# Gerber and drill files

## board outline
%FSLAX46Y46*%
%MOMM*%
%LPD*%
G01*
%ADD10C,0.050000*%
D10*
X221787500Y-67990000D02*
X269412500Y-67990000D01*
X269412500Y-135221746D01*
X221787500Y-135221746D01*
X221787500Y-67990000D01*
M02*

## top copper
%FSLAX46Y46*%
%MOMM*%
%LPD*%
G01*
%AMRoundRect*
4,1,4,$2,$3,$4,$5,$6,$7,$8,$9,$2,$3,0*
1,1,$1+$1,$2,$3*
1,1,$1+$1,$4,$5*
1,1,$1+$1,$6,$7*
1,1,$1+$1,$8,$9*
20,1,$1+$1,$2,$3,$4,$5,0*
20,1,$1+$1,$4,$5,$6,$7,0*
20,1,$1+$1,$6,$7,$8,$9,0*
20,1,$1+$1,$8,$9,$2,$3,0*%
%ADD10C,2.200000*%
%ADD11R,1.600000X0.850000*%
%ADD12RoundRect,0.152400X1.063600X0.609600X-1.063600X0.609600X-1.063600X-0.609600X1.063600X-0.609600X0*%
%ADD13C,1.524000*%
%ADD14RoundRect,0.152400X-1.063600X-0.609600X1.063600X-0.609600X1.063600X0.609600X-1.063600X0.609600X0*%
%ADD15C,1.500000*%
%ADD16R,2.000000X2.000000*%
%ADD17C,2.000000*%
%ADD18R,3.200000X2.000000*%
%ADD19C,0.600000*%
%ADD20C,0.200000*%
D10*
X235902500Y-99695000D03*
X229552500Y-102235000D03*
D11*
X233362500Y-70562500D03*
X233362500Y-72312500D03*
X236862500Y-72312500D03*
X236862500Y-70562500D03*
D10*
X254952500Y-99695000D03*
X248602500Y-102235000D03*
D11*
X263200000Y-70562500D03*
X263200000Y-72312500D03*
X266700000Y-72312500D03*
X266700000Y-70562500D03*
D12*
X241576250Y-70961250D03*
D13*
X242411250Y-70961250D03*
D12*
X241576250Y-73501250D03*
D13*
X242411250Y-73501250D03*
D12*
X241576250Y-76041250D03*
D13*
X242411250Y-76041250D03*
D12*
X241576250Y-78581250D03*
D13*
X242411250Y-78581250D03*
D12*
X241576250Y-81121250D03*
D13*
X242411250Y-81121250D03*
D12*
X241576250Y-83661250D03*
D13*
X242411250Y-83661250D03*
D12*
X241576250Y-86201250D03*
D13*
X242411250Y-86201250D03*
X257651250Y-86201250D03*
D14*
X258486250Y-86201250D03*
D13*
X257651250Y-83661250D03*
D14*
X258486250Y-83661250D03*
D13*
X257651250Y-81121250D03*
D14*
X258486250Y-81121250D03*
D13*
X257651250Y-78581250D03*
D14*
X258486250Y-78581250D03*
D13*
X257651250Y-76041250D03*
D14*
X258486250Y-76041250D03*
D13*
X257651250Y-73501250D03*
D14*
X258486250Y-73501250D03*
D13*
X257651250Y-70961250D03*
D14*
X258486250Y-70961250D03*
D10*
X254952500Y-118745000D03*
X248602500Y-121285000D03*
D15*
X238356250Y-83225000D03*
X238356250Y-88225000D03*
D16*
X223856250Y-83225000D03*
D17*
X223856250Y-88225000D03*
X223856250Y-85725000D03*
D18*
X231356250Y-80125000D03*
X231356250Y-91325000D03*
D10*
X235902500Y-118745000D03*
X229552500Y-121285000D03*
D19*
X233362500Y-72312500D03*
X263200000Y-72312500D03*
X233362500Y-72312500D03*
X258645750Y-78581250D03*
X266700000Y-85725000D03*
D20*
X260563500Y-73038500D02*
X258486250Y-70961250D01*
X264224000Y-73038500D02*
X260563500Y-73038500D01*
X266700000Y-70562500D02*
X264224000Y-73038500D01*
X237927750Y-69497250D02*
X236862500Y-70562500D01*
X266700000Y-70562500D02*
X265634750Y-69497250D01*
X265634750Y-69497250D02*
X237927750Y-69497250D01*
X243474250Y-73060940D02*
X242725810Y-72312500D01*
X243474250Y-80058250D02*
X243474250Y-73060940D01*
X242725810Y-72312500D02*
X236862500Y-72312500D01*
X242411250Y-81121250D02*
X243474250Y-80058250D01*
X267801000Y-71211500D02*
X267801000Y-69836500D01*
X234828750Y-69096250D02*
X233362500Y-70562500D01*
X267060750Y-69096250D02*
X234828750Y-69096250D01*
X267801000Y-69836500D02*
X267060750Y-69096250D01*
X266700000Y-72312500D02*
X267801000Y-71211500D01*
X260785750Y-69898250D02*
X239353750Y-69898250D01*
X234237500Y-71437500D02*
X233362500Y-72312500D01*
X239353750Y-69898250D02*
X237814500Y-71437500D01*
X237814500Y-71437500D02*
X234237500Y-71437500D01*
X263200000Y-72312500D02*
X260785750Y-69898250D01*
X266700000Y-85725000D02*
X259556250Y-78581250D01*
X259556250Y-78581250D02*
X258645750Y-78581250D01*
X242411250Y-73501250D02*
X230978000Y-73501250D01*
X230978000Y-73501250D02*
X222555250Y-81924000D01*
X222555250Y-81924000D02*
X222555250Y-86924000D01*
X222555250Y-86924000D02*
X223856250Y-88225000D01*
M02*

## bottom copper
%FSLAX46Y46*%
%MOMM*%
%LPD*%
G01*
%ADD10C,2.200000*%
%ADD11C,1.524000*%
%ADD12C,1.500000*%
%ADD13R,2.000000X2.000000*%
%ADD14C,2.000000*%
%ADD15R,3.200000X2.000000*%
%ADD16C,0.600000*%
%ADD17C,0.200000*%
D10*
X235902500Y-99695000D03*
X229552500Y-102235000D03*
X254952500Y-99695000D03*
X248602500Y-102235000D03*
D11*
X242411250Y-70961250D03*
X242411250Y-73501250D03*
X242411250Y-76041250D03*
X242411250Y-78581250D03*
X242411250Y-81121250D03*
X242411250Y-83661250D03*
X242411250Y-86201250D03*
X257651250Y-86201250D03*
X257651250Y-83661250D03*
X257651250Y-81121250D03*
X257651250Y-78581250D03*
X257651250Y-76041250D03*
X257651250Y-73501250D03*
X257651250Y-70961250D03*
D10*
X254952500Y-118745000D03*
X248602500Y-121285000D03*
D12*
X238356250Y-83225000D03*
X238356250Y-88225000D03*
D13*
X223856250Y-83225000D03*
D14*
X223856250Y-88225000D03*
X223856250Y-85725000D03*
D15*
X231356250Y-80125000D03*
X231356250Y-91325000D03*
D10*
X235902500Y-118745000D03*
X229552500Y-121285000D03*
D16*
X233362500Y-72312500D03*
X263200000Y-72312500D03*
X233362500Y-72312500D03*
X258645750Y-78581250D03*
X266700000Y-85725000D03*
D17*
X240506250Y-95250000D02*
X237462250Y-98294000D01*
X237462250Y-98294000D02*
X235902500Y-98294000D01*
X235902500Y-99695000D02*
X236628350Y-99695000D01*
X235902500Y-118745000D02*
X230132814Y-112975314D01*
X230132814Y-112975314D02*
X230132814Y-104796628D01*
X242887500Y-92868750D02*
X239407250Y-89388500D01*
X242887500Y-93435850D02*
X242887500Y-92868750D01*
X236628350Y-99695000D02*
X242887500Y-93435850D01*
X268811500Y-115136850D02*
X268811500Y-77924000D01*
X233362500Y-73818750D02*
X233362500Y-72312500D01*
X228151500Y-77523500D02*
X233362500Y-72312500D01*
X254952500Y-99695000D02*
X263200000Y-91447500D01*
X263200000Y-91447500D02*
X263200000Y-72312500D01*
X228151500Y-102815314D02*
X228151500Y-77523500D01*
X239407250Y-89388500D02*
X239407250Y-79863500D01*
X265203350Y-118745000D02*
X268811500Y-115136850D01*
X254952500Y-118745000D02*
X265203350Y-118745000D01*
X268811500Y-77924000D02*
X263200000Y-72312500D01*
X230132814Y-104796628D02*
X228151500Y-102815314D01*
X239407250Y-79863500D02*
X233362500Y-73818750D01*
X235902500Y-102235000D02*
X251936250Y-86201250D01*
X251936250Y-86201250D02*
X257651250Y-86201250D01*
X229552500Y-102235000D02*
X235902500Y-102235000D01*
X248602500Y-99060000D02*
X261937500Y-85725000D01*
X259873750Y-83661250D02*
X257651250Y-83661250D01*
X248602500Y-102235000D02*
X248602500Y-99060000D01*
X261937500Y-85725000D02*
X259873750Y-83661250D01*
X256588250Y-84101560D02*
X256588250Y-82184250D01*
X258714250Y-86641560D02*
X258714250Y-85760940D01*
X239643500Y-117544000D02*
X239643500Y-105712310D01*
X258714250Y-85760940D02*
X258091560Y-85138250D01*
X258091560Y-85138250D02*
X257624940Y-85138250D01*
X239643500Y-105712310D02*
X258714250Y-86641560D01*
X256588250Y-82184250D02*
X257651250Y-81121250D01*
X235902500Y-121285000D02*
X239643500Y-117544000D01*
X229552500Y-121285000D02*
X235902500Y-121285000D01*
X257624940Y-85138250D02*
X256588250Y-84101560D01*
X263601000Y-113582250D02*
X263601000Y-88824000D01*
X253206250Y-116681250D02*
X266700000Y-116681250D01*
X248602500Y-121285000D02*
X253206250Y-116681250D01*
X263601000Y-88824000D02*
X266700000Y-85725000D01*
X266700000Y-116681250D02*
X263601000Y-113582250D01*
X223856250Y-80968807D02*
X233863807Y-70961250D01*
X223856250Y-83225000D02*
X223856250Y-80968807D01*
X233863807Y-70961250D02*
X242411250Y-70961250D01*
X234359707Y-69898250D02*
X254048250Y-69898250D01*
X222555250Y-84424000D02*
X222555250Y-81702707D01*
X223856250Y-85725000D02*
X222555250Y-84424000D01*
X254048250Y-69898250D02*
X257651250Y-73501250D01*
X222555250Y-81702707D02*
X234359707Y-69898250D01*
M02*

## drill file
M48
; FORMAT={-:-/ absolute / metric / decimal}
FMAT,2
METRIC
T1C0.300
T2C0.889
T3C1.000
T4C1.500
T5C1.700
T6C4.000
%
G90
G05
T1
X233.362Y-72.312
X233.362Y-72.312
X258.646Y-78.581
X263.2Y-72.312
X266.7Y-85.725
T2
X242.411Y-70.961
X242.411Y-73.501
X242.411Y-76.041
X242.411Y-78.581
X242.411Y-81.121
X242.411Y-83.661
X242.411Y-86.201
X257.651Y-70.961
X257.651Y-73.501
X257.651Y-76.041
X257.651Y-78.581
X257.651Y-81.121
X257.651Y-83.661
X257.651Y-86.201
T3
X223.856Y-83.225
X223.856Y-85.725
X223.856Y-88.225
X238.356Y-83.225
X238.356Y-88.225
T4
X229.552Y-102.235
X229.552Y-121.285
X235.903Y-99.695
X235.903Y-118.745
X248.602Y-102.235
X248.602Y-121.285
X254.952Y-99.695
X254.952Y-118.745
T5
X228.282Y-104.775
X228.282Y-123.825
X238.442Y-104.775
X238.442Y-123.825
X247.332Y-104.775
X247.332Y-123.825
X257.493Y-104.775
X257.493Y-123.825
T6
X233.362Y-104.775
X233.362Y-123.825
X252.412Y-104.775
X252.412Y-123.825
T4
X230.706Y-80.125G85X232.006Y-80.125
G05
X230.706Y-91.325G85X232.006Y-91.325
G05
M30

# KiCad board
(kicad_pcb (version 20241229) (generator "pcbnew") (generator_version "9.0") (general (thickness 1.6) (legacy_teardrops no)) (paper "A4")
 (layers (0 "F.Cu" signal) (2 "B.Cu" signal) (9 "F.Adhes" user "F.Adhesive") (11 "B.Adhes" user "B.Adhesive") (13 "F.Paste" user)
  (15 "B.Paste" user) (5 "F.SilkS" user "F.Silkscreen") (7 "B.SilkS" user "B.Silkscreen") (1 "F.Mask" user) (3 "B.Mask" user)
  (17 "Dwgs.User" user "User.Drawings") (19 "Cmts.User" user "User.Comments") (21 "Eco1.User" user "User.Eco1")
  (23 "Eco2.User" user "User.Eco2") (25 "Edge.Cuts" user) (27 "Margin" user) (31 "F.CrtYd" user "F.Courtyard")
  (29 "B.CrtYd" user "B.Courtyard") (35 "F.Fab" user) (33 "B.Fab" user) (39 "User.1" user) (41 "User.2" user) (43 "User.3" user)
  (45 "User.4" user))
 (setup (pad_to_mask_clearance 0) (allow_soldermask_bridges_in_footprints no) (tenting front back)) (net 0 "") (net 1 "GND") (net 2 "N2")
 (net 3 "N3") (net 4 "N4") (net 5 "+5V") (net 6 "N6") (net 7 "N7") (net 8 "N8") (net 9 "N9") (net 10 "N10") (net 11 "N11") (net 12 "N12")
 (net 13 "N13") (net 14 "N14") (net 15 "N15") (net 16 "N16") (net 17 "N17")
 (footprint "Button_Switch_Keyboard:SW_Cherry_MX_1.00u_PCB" (layer "F.Cu") (at 235.9025 99.695)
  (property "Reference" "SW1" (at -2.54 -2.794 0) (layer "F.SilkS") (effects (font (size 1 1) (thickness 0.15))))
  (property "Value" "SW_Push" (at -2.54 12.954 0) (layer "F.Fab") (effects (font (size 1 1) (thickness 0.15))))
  (pad "" np_thru_hole circle (at -7.62 5.08) (size 1.7 1.7) (drill 1.7) (layers "*.Cu" "*.Mask"))
  (pad "" np_thru_hole circle (at -2.54 5.08) (size 4 4) (drill 4) (layers "*.Cu" "*.Mask"))
  (pad "" np_thru_hole circle (at 2.54 5.08) (size 1.7 1.7) (drill 1.7) (layers "*.Cu" "*.Mask"))
  (pad "1" thru_hole circle (at 0 0) (size 2.2 2.2) (drill 1.5) (layers "*.Cu" "*.Mask") (remove_unused_layers no) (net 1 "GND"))
  (pad "2" thru_hole circle (at -6.35 2.54) (size 2.2 2.2) (drill 1.5) (layers "*.Cu" "*.Mask") (remove_unused_layers no) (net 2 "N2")))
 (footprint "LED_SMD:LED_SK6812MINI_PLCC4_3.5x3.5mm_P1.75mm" (layer "F.Cu") (at 235.1125 71.4375)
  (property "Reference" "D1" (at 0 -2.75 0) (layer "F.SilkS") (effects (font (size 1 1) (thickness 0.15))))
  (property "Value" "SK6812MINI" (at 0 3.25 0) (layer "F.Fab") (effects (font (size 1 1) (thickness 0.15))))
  (pad "1" smd rect (at -1.75 -0.875) (size 1.6 0.85) (layers "F.Cu" "F.Mask" "F.Paste") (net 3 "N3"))
  (pad "2" smd rect (at -1.75 0.875) (size 1.6 0.85) (layers "F.Cu" "F.Mask" "F.Paste") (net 1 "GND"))
  (pad "3" smd rect (at 1.75 0.875) (size 1.6 0.85) (layers "F.Cu" "F.Mask" "F.Paste") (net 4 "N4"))
  (pad "4" smd rect (at 1.75 -0.875) (size 1.6 0.85) (layers "F.Cu" "F.Mask" "F.Paste") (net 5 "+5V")))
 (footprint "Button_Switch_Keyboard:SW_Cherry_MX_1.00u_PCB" (layer "F.Cu") (at 254.9525 99.695)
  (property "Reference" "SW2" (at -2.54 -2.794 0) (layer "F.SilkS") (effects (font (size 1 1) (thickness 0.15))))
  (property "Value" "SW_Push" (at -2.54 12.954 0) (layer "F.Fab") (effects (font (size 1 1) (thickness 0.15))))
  (pad "" np_thru_hole circle (at -7.62 5.08) (size 1.7 1.7) (drill 1.7) (layers "*.Cu" "*.Mask"))
  (pad "" np_thru_hole circle (at -2.54 5.08) (size 4 4) (drill 4) (layers "*.Cu" "*.Mask"))
  (pad "" np_thru_hole circle (at 2.54 5.08) (size 1.7 1.7) (drill 1.7) (layers "*.Cu" "*.Mask"))
  (pad "1" thru_hole circle (at 0 0) (size 2.2 2.2) (drill 1.5) (layers "*.Cu" "*.Mask") (remove_unused_layers no) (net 1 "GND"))
  (pad "2" thru_hole circle (at -6.35 2.54) (size 2.2 2.2) (drill 1.5) (layers "*.Cu" "*.Mask") (remove_unused_layers no) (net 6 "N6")))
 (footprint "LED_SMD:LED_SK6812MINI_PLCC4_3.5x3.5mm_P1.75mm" (layer "F.Cu") (at 264.95 71.4375)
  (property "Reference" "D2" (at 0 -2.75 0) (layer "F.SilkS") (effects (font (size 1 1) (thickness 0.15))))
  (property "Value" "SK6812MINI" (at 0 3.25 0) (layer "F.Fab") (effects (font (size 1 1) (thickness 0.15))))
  (pad "1" smd rect (at -1.75 -0.875) (size 1.6 0.85) (layers "F.Cu" "F.Mask" "F.Paste") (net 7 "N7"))
  (pad "2" smd rect (at -1.75 0.875) (size 1.6 0.85) (layers "F.Cu" "F.Mask" "F.Paste") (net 1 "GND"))
  (pad "3" smd rect (at 1.75 0.875) (size 1.6 0.85) (layers "F.Cu" "F.Mask" "F.Paste") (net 3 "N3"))
  (pad "4" smd rect (at 1.75 -0.875) (size 1.6 0.85) (layers "F.Cu" "F.Mask" "F.Paste") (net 5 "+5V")))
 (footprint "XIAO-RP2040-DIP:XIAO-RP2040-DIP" (layer "F.Cu") (at 250.03125 78.58125)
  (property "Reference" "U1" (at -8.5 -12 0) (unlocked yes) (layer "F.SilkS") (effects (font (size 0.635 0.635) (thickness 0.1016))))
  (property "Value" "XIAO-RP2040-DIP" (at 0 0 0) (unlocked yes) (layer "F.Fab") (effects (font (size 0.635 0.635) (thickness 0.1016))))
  (pad "1" smd roundrect (at -8.455 -7.62 180) (size 2.432 1.524) (layers "F.Cu" "F.Mask") (roundrect_rratio 0.1) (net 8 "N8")
   (thermal_bridge_angle 45))
  (pad "1" thru_hole circle (at -7.62 -7.62 180) (size 1.524 1.524) (drill 0.889) (layers "*.Cu" "*.Mask") (remove_unused_layers no)
   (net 8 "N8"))
  (pad "2" smd roundrect (at -8.455 -5.08 180) (size 2.432 1.524) (layers "F.Cu" "F.Mask") (roundrect_rratio 0.1) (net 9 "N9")
   (thermal_bridge_angle 45))
  (pad "2" thru_hole circle (at -7.62 -5.08 180) (size 1.524 1.524) (drill 0.889) (layers "*.Cu" "*.Mask") (remove_unused_layers no)
   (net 9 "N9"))
  (pad "3" smd roundrect (at -8.455 -2.54 180) (size 2.432 1.524) (layers "F.Cu" "F.Mask") (roundrect_rratio 0.1) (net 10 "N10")
   (thermal_bridge_angle 45))
  (pad "3" thru_hole circle (at -7.62 -2.54 180) (size 1.524 1.524) (drill 0.889) (layers "*.Cu" "*.Mask") (remove_unused_layers no)
   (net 10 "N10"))
  (pad "4" smd roundrect (at -8.455 0 180) (size 2.432 1.524) (layers "F.Cu" "F.Mask") (roundrect_rratio 0.1) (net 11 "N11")
   (thermal_bridge_angle 45))
  (pad "4" thru_hole circle (at -7.62 0 180) (size 1.524 1.524) (drill 0.889) (layers "*.Cu" "*.Mask") (remove_unused_layers no)
   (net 11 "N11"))
  (pad "5" smd roundrect (at -8.455 2.54 180) (size 2.432 1.524) (layers "F.Cu" "F.Mask") (roundrect_rratio 0.1) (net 4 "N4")
   (thermal_bridge_angle 45))
  (pad "5" thru_hole circle (at -7.62 2.54 180) (size 1.524 1.524) (drill 0.889) (layers "*.Cu" "*.Mask") (remove_unused_layers no)
   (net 4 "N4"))
  (pad "6" smd roundrect (at -8.455 5.08 180) (size 2.432 1.524) (layers "F.Cu" "F.Mask") (roundrect_rratio 0.1) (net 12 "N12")
   (thermal_bridge_angle 45))
  (pad "6" thru_hole circle (at -7.62 5.08 180) (size 1.524 1.524) (drill 0.889) (layers "*.Cu" "*.Mask") (remove_unused_layers no)
   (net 12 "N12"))
  (pad "7" smd roundrect (at -8.455 7.62 180) (size 2.432 1.524) (layers "F.Cu" "F.Mask") (roundrect_rratio 0.1) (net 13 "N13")
   (thermal_bridge_angle 45))
  (pad "7" thru_hole circle (at -7.62 7.62 180) (size 1.524 1.524) (drill 0.889) (layers "*.Cu" "*.Mask") (remove_unused_layers no)
   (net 13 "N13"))
  (pad "8" thru_hole circle (at 7.62 7.62) (size 1.524 1.524) (drill 0.889) (layers "*.Cu" "*.Mask") (remove_unused_layers no) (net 2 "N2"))
  (pad "8" smd roundrect (at 8.455 7.62) (size 2.432 1.524) (layers "F.Cu" "F.Mask") (roundrect_rratio 0.1) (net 2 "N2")
   (thermal_bridge_angle 45))
  (pad "9" thru_hole circle (at 7.62 5.08) (size 1.524 1.524) (drill 0.889) (layers "*.Cu" "*.Mask") (remove_unused_layers no) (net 6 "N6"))
  (pad "9" smd roundrect (at 8.455 5.08) (size 2.432 1.524) (layers "F.Cu" "F.Mask") (roundrect_rratio 0.1) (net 6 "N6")
   (thermal_bridge_angle 45))
  (pad "10" thru_hole circle (at 7.62 2.54) (size 1.524 1.524) (drill 0.889) (layers "*.Cu" "*.Mask") (remove_unused_layers no)
   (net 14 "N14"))
  (pad "10" smd roundrect (at 8.455 2.54) (size 2.432 1.524) (layers "F.Cu" "F.Mask") (roundrect_rratio 0.1) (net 14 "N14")
   (thermal_bridge_angle 45))
  (pad "11" thru_hole circle (at 7.62 0) (size 1.524 1.524) (drill 0.889) (layers "*.Cu" "*.Mask") (remove_unused_layers no) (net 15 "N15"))
  (pad "11" smd roundrect (at 8.455 0) (size 2.432 1.524) (layers "F.Cu" "F.Mask") (roundrect_rratio 0.1) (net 15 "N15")
   (thermal_bridge_angle 45))
  (pad "12" thru_hole circle (at 7.62 -2.54) (size 1.524 1.524) (drill 0.889) (layers "*.Cu" "*.Mask") (remove_unused_layers no)
   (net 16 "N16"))
  (pad "12" smd roundrect (at 8.455 -2.54) (size 2.432 1.524) (layers "F.Cu" "F.Mask") (roundrect_rratio 0.1) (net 16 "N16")
   (thermal_bridge_angle 45))
  (pad "13" thru_hole circle (at 7.62 -5.08) (size 1.524 1.524) (drill 0.889) (layers "*.Cu" "*.Mask") (remove_unused_layers no)
   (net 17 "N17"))
  (pad "13" smd roundrect (at 8.455 -5.08) (size 2.432 1.524) (layers "F.Cu" "F.Mask") (roundrect_rratio 0.1) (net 17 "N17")
   (thermal_bridge_angle 45))
  (pad "14" thru_hole circle (at 7.62 -7.62) (size 1.524 1.524) (drill 0.889) (layers "*.Cu" "*.Mask") (remove_unused_layers no)
   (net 5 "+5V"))
  (pad "14" smd roundrect (at 8.455 -7.62) (size 2.432 1.524) (layers "F.Cu" "F.Mask") (roundrect_rratio 0.1) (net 5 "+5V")
   (thermal_bridge_angle 45)))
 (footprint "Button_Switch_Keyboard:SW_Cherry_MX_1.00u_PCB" (layer "F.Cu") (at 254.9525 118.745)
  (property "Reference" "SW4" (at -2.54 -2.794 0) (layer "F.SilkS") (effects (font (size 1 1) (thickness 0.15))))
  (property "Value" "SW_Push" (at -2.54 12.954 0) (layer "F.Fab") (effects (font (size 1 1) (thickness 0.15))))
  (pad "" np_thru_hole circle (at -7.62 5.08) (size 1.7 1.7) (drill 1.7) (layers "*.Cu" "*.Mask"))
  (pad "" np_thru_hole circle (at -2.54 5.08) (size 4 4) (drill 4) (layers "*.Cu" "*.Mask"))
  (pad "" np_thru_hole circle (at 2.54 5.08) (size 1.7 1.7) (drill 1.7) (layers "*.Cu" "*.Mask"))
  (pad "1" thru_hole circle (at 0 0) (size 2.2 2.2) (drill 1.5) (layers "*.Cu" "*.Mask") (remove_unused_layers no) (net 1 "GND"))
  (pad "2" thru_hole circle (at -6.35 2.54) (size 2.2 2.2) (drill 1.5) (layers "*.Cu" "*.Mask") (remove_unused_layers no) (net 15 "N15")))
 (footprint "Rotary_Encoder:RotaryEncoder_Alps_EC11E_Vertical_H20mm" (layer "F.Cu") (at 223.85625 83.225)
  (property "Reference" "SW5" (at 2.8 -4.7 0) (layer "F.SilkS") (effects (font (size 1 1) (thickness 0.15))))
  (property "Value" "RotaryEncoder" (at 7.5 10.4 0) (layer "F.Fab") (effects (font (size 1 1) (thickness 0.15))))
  (pad "" thru_hole circle (at 14.5 0) (size 1.5 1.5) (drill 1) (layers "*.Cu" "*.Mask") (remove_unused_layers no))
  (pad "" thru_hole circle (at 14.5 5) (size 1.5 1.5) (drill 1) (layers "*.Cu" "*.Mask") (remove_unused_layers no))
  (pad "A" thru_hole rect (at 0 0) (size 2 2) (drill 1) (layers "*.Cu" "*.Mask") (remove_unused_layers no) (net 8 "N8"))
  (pad "B" thru_hole circle (at 0 5) (size 2 2) (drill 1) (layers "*.Cu" "*.Mask") (remove_unused_layers no) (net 9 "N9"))
  (pad "C" thru_hole circle (at 0 2.5) (size 2 2) (drill 1) (layers "*.Cu" "*.Mask") (remove_unused_layers no) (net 17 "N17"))
  (pad "MP" thru_hole rect (at 7.5 -3.1) (size 3.2 2) (drill oval 2.8 1.5) (layers "*.Cu" "*.Mask") (remove_unused_layers no))
  (pad "MP" thru_hole rect (at 7.5 8.1) (size 3.2 2) (drill oval 2.8 1.5) (layers "*.Cu" "*.Mask") (remove_unused_layers no)))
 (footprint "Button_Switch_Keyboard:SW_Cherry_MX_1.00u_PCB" (layer "F.Cu") (at 235.9025 118.745)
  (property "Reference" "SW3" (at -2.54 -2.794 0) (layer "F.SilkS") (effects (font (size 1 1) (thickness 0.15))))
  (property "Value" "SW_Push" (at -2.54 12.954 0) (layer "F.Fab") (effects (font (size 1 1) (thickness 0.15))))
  (pad "" np_thru_hole circle (at -7.62 5.08) (size 1.7 1.7) (drill 1.7) (layers "*.Cu" "*.Mask"))
  (pad "" np_thru_hole circle (at -2.54 5.08) (size 4 4) (drill 4) (layers "*.Cu" "*.Mask"))
  (pad "" np_thru_hole circle (at 2.54 5.08) (size 1.7 1.7) (drill 1.7) (layers "*.Cu" "*.Mask"))
  (pad "1" thru_hole circle (at 0 0) (size 2.2 2.2) (drill 1.5) (layers "*.Cu" "*.Mask") (remove_unused_layers no) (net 1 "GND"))
  (pad "2" thru_hole circle (at -6.35 2.54) (size 2.2 2.2) (drill 1.5) (layers "*.Cu" "*.Mask") (remove_unused_layers no) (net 14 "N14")))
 (gr_rect (start 221.7875 67.99) (end 269.4125 135.221746) (stroke (width 0.05) (type default)) (fill no) (layer "Edge.Cuts"))
 (segment (start 240.50625 95.25) (end 237.46225 98.294) (width 0.2) (layer "B.Cu") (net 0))
 (segment (start 237.46225 98.294) (end 235.9025 98.294) (width 0.2) (layer "B.Cu") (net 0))
 (segment (start 260.5635 73.0385) (end 258.48625 70.96125) (width 0.2) (layer "F.Cu") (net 5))
 (segment (start 264.224 73.0385) (end 260.5635 73.0385) (width 0.2) (layer "F.Cu") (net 5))
 (segment (start 266.7 70.5625) (end 264.224 73.0385) (width 0.2) (layer "F.Cu") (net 5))
 (segment (start 237.92775 69.49725) (end 236.8625 70.5625) (width 0.2) (layer "F.Cu") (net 5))
 (segment (start 266.7 70.5625) (end 265.63475 69.49725) (width 0.2) (layer "F.Cu") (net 5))
 (segment (start 265.63475 69.49725) (end 237.92775 69.49725) (width 0.2) (layer "F.Cu") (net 5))
 (segment (start 243.47425 73.06094) (end 242.72581 72.3125) (width 0.2) (layer "F.Cu") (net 4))
 (segment (start 243.47425 80.05825) (end 243.47425 73.06094) (width 0.2) (layer "F.Cu") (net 4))
 (segment (start 242.72581 72.3125) (end 236.8625 72.3125) (width 0.2) (layer "F.Cu") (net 4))
 (segment (start 242.41125 81.12125) (end 243.47425 80.05825) (width 0.2) (layer "F.Cu") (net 4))
 (segment (start 267.801 71.2115) (end 267.801 69.8365) (width 0.2) (layer "F.Cu") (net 3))
 (segment (start 234.82875 69.09625) (end 233.3625 70.5625) (width 0.2) (layer "F.Cu") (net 3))
 (segment (start 267.06075 69.09625) (end 234.82875 69.09625) (width 0.2) (layer "F.Cu") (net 3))
 (segment (start 267.801 69.8365) (end 267.06075 69.09625) (width 0.2) (layer "F.Cu") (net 3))
 (segment (start 266.7 72.3125) (end 267.801 71.2115) (width 0.2) (layer "F.Cu") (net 3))
 (segment (start 260.78575 69.89825) (end 239.35375 69.89825) (width 0.2) (layer "F.Cu") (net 1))
 (segment (start 234.2375 71.4375) (end 233.3625 72.3125) (width 0.2) (layer "F.Cu") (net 1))
 (segment (start 239.35375 69.89825) (end 237.8145 71.4375) (width 0.2) (layer "F.Cu") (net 1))
 (segment (start 237.8145 71.4375) (end 234.2375 71.4375) (width 0.2) (layer "F.Cu") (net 1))
 (segment (start 263.2 72.3125) (end 260.78575 69.89825) (width 0.2) (layer "F.Cu") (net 1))
 (via (at 233.3625 72.3125) (size 0.6) (drill 0.3) (layers "F.Cu" "B.Cu") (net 1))
 (via (at 263.2 72.3125) (size 0.6) (drill 0.3) (layers "F.Cu" "B.Cu") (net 1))
 (via (at 233.3625 72.3125) (size 0.6) (drill 0.3) (layers "F.Cu" "B.Cu") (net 1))
 (segment (start 235.9025 99.695) (end 236.62835 99.695) (width 0.2) (layer "B.Cu") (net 1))
 (segment (start 235.9025 118.745) (end 230.132814 112.975314) (width 0.2) (layer "B.Cu") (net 1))
 (segment (start 230.132814 112.975314) (end 230.132814 104.796628) (width 0.2) (layer "B.Cu") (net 1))
 (segment (start 242.8875 92.86875) (end 239.40725 89.3885) (width 0.2) (layer "B.Cu") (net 1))
 (segment (start 242.8875 93.43585) (end 242.8875 92.86875) (width 0.2) (layer "B.Cu") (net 1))
 (segment (start 236.62835 99.695) (end 242.8875 93.43585) (width 0.2) (layer "B.Cu") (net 1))
 (segment (start 268.8115 115.13685) (end 268.8115 77.924) (width 0.2) (layer "B.Cu") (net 1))
 (segment (start 233.3625 73.81875) (end 233.3625 72.3125) (width 0.2) (layer "B.Cu") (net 1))
 (segment (start 228.1515 77.5235) (end 233.3625 72.3125) (width 0.2) (layer "B.Cu") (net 1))
 (segment (start 254.9525 99.695) (end 263.2 91.4475) (width 0.2) (layer "B.Cu") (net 1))
 (segment (start 263.2 91.4475) (end 263.2 72.3125) (width 0.2) (layer "B.Cu") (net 1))
 (segment (start 228.1515 102.815314) (end 228.1515 77.5235) (width 0.2) (layer "B.Cu") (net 1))
 (segment (start 239.40725 89.3885) (end 239.40725 79.8635) (width 0.2) (layer "B.Cu") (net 1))
 (segment (start 265.20335 118.745) (end 268.8115 115.13685) (width 0.2) (layer "B.Cu") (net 1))
 (segment (start 254.9525 118.745) (end 265.20335 118.745) (width 0.2) (layer "B.Cu") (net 1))
 (segment (start 268.8115 77.924) (end 263.2 72.3125) (width 0.2) (layer "B.Cu") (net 1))
 (segment (start 230.132814 104.796628) (end 228.1515 102.815314) (width 0.2) (layer "B.Cu") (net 1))
 (segment (start 239.40725 79.8635) (end 233.3625 73.81875) (width 0.2) (layer "B.Cu") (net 1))
 (segment (start 235.9025 102.235) (end 251.93625 86.20125) (width 0.2) (layer "B.Cu") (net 2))
 (segment (start 251.93625 86.20125) (end 257.65125 86.20125) (width 0.2) (layer "B.Cu") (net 2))
 (segment (start 229.5525 102.235) (end 235.9025 102.235) (width 0.2) (layer "B.Cu") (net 2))
 (segment (start 248.6025 99.06) (end 261.9375 85.725) (width 0.2) (layer "B.Cu") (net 6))
 (segment (start 259.87375 83.66125) (end 257.65125 83.66125) (width 0.2) (layer "B.Cu") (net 6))
 (segment (start 248.6025 102.235) (end 248.6025 99.06) (width 0.2) (layer "B.Cu") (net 6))
 (segment (start 261.9375 85.725) (end 259.87375 83.66125) (width 0.2) (layer "B.Cu") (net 6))
 (segment (start 256.58825 84.10156) (end 256.58825 82.18425) (width 0.2) (layer "B.Cu") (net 14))
 (segment (start 258.71425 86.64156) (end 258.71425 85.76094) (width 0.2) (layer "B.Cu") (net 14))
 (segment (start 239.6435 117.544) (end 239.6435 105.71231) (width 0.2) (layer "B.Cu") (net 14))
 (segment (start 258.71425 85.76094) (end 258.09156 85.13825) (width 0.2) (layer "B.Cu") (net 14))
 (segment (start 258.09156 85.13825) (end 257.62494 85.13825) (width 0.2) (layer "B.Cu") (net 14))
 (segment (start 239.6435 105.71231) (end 258.71425 86.64156) (width 0.2) (layer "B.Cu") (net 14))
 (segment (start 256.58825 82.18425) (end 257.65125 81.12125) (width 0.2) (layer "B.Cu") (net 14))
 (segment (start 235.9025 121.285) (end 239.6435 117.544) (width 0.2) (layer "B.Cu") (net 14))
 (segment (start 229.5525 121.285) (end 235.9025 121.285) (width 0.2) (layer "B.Cu") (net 14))
 (segment (start 257.62494 85.13825) (end 256.58825 84.10156) (width 0.2) (layer "B.Cu") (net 14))
 (segment (start 266.7 85.725) (end 259.55625 78.58125) (width 0.2) (layer "F.Cu") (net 15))
 (segment (start 259.55625 78.58125) (end 258.64575 78.58125) (width 0.2) (layer "F.Cu") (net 15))
 (via (at 258.64575 78.58125) (size 0.6) (drill 0.3) (layers "F.Cu" "B.Cu") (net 15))
 (via (at 266.7 85.725) (size 0.6) (drill 0.3) (layers "F.Cu" "B.Cu") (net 15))
 (segment (start 263.601 113.58225) (end 263.601 88.824) (width 0.2) (layer "B.Cu") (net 15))
 (segment (start 253.20625 116.68125) (end 266.7 116.68125) (width 0.2) (layer "B.Cu") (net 15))
 (segment (start 248.6025 121.285) (end 253.20625 116.68125) (width 0.2) (layer "B.Cu") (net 15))
 (segment (start 263.601 88.824) (end 266.7 85.725) (width 0.2) (layer "B.Cu") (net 15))
 (segment (start 266.7 116.68125) (end 263.601 113.58225) (width 0.2) (layer "B.Cu") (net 15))
 (segment (start 223.85625 80.968807) (end 233.863807 70.96125) (width 0.2) (layer "B.Cu") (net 8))
 (segment (start 223.85625 83.225) (end 223.85625 80.968807) (width 0.2) (layer "B.Cu") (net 8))
 (segment (start 233.863807 70.96125) (end 242.41125 70.96125) (width 0.2) (layer "B.Cu") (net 8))
 (segment (start 242.41125 73.50125) (end 230.978 73.50125) (width 0.2) (layer "F.Cu") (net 9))
 (segment (start 230.978 73.50125) (end 222.55525 81.924) (width 0.2) (layer "F.Cu") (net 9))
 (segment (start 222.55525 81.924) (end 222.55525 86.924) (width 0.2) (layer "F.Cu") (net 9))
 (segment (start 222.55525 86.924) (end 223.85625 88.225) (width 0.2) (layer "F.Cu") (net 9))
 (segment (start 234.359707 69.89825) (end 254.04825 69.89825) (width 0.2) (layer "B.Cu") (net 17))
 (segment (start 222.55525 84.424) (end 222.55525 81.702707) (width 0.2) (layer "B.Cu") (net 17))
 (segment (start 223.85625 85.725) (end 222.55525 84.424) (width 0.2) (layer "B.Cu") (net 17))
 (segment (start 254.04825 69.89825) (end 257.65125 73.50125) (width 0.2) (layer "B.Cu") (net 17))
 (segment (start 222.55525 81.702707) (end 234.359707 69.89825) (width 0.2) (layer "B.Cu") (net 17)))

